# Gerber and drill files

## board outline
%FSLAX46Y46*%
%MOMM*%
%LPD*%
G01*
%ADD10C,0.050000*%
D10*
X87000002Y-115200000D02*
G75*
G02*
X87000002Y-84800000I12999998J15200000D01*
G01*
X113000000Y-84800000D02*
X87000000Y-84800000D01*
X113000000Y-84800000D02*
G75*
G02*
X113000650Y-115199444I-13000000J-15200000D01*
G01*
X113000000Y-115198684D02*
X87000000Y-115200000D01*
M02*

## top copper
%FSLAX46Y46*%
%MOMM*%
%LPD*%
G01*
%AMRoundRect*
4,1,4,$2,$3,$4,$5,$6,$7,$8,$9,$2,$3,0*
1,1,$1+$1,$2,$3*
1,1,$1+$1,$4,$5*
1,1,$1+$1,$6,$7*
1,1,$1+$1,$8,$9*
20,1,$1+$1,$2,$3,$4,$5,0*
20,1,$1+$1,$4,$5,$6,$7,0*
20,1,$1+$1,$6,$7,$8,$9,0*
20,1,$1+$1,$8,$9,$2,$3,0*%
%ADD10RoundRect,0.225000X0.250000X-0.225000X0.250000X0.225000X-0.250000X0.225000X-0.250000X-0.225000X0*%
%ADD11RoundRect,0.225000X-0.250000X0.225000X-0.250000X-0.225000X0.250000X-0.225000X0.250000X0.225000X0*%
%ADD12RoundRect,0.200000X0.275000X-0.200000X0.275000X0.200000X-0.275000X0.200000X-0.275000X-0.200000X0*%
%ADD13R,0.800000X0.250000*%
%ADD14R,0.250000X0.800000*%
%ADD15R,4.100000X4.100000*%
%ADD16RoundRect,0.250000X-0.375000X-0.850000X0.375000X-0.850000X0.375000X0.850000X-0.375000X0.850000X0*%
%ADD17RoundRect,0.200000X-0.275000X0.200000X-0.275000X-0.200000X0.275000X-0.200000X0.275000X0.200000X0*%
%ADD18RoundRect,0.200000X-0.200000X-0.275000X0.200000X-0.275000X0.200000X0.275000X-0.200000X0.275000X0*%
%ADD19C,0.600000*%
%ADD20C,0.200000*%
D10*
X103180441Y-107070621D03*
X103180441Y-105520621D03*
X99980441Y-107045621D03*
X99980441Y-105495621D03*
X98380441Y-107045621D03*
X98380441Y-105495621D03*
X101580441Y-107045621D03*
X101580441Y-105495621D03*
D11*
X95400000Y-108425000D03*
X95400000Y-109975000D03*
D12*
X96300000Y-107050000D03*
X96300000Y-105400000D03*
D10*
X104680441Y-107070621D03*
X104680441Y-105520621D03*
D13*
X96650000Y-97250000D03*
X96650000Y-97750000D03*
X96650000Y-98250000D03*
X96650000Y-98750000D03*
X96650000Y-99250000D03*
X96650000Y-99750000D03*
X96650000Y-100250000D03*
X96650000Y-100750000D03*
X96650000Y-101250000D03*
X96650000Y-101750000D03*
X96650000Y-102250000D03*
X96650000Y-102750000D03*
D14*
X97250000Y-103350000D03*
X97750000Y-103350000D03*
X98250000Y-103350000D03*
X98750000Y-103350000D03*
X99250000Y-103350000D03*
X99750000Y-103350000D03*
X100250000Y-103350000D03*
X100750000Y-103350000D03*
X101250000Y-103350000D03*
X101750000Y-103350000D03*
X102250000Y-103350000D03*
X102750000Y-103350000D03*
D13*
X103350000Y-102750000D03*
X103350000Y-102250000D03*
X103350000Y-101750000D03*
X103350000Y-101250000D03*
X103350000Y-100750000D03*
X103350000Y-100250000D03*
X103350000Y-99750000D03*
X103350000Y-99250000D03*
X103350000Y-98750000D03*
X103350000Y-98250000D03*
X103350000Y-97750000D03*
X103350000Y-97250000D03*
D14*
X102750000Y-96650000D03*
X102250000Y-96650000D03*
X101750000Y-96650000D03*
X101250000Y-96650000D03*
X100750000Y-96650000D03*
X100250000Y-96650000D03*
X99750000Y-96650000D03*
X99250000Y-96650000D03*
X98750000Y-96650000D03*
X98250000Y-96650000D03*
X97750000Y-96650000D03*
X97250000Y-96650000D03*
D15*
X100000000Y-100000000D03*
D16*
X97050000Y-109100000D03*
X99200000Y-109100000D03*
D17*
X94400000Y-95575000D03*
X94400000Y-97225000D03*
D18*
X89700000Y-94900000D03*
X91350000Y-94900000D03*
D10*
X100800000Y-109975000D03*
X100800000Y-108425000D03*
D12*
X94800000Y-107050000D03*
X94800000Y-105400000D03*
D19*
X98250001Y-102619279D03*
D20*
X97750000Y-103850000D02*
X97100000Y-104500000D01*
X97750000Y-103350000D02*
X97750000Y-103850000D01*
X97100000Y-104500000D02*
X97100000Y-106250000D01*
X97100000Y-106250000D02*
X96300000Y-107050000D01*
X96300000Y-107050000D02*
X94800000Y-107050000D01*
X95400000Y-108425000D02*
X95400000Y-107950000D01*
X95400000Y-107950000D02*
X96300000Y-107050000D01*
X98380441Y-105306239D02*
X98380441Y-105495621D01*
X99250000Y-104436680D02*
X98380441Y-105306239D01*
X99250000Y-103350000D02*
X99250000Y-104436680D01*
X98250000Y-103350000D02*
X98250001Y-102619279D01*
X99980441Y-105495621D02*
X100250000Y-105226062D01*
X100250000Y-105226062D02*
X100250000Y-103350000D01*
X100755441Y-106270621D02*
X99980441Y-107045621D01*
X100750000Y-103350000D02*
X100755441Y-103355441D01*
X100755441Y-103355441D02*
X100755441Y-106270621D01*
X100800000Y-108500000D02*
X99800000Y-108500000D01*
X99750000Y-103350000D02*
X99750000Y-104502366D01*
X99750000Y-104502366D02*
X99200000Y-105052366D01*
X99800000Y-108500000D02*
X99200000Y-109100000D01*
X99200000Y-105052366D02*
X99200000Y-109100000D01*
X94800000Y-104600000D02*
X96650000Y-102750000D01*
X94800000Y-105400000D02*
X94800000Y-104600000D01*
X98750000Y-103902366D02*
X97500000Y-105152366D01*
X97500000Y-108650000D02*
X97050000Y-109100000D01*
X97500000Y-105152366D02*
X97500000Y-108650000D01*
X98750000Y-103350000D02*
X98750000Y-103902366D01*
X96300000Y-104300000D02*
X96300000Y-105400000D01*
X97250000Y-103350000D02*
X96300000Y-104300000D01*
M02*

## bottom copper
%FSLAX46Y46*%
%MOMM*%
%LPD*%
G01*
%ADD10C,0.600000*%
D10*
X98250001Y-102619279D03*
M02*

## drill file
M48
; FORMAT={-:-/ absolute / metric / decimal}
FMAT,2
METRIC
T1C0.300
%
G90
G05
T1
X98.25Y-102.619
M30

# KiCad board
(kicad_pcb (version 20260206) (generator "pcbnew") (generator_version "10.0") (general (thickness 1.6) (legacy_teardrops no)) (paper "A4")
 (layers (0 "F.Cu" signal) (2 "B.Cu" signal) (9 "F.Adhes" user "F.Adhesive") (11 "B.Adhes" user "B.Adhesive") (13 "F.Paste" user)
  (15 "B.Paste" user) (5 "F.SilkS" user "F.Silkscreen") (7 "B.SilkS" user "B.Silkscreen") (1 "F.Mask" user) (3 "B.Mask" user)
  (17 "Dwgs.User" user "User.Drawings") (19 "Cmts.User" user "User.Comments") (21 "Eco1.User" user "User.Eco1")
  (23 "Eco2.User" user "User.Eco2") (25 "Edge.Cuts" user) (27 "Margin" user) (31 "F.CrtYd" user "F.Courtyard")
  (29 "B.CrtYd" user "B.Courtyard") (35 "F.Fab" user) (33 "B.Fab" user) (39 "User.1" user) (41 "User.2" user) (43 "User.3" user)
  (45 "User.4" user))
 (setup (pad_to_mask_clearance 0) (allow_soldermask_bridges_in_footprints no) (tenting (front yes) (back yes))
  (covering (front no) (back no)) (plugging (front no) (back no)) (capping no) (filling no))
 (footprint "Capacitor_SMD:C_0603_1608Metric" (layer "F.Cu") (at 103.180441 106.295621 90)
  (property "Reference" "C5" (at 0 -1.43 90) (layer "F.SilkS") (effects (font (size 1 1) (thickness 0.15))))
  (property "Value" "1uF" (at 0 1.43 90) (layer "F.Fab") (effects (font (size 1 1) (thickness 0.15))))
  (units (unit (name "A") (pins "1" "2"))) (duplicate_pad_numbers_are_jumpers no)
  (pad "1" smd roundrect (at -0.775 0 90) (size 0.9 0.95) (layers "F.Cu" "F.Mask" "F.Paste") (roundrect_rratio 0.25) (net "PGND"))
  (pad "2" smd roundrect (at 0.775 0 90) (size 0.9 0.95) (layers "F.Cu" "F.Mask" "F.Paste") (roundrect_rratio 0.25) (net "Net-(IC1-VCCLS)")))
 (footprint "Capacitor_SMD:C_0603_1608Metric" (layer "F.Cu") (at 99.980441 106.270621 90)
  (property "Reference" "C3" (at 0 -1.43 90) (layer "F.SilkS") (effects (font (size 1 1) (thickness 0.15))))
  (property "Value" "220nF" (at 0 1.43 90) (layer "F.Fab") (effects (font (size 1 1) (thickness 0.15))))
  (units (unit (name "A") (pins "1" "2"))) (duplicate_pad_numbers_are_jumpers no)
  (pad "1" smd roundrect (at -0.775 0 90) (size 0.9 0.95) (layers "F.Cu" "F.Mask" "F.Paste") (roundrect_rratio 0.25) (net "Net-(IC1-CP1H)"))
  (pad "2" smd roundrect (at 0.775 0 90) (size 0.9 0.95) (layers "F.Cu" "F.Mask" "F.Paste") (roundrect_rratio 0.25) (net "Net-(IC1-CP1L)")))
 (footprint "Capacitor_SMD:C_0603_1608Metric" (layer "F.Cu") (at 98.380441 106.270621 90)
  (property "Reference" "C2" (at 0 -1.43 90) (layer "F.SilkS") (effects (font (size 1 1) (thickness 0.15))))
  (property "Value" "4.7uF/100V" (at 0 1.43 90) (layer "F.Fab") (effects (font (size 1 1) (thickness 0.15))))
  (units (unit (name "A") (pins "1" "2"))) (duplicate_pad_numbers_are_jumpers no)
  (pad "1" smd roundrect (at -0.775 0 90) (size 0.9 0.95) (layers "F.Cu" "F.Mask" "F.Paste") (roundrect_rratio 0.25) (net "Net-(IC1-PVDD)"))
  (pad "2" smd roundrect (at 0.775 0 90) (size 0.9 0.95) (layers "F.Cu" "F.Mask" "F.Paste") (roundrect_rratio 0.25) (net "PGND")))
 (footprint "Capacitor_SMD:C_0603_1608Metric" (layer "F.Cu") (at 101.580441 106.270621 90)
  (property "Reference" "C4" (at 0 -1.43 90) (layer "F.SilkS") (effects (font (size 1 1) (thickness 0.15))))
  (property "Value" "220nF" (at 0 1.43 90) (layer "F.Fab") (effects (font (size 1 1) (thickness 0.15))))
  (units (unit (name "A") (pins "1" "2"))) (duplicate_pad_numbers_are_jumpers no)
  (pad "1" smd roundrect (at -0.775 0 90) (size 0.9 0.95) (layers "F.Cu" "F.Mask" "F.Paste") (roundrect_rratio 0.25) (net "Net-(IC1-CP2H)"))
  (pad "2" smd roundrect (at 0.775 0 90) (size 0.9 0.95) (layers "F.Cu" "F.Mask" "F.Paste") (roundrect_rratio 0.25) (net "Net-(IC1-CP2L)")))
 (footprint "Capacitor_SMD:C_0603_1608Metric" (layer "F.Cu") (at 95.4 109.2 -90)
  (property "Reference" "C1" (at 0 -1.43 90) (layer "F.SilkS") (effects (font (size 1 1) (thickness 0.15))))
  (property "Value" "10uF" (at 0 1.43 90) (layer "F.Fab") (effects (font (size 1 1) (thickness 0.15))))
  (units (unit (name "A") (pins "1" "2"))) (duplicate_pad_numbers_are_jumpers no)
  (pad "1" smd roundrect (at -0.775 0 270) (size 0.9 0.95) (layers "F.Cu" "F.Mask" "F.Paste") (roundrect_rratio 0.25) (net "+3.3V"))
  (pad "2" smd roundrect (at 0.775 0 270) (size 0.9 0.95) (layers "F.Cu" "F.Mask" "F.Paste") (roundrect_rratio 0.25) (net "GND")))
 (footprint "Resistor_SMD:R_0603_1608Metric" (layer "F.Cu") (at 96.3 106.225 90)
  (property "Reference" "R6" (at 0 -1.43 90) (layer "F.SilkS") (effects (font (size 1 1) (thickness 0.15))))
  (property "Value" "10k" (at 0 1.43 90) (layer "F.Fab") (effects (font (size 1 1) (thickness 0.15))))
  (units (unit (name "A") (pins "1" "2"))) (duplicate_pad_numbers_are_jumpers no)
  (pad "1" smd roundrect (at -0.825 0 90) (size 0.8 0.95) (layers "F.Cu" "F.Mask" "F.Paste") (roundrect_rratio 0.25) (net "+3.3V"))
  (pad "2" smd roundrect (at 0.825 0 90) (size 0.8 0.95) (layers "F.Cu" "F.Mask" "F.Paste") (roundrect_rratio 0.25) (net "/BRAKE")))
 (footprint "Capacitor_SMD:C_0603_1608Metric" (layer "F.Cu") (at 104.680441 106.295621 90)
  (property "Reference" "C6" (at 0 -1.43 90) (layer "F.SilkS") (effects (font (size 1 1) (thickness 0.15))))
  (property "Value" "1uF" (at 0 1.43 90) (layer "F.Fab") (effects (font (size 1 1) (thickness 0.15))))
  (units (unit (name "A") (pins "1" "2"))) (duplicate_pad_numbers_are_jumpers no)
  (pad "1" smd roundrect (at -0.775 0 90) (size 0.9 0.95) (layers "F.Cu" "F.Mask" "F.Paste") (roundrect_rratio 0.25) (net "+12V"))
  (pad "2" smd roundrect (at 0.775 0 90) (size 0.9 0.95) (layers "F.Cu" "F.Mask" "F.Paste") (roundrect_rratio 0.25) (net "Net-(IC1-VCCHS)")))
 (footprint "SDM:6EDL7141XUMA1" (layer "F.Cu") (at 100 100)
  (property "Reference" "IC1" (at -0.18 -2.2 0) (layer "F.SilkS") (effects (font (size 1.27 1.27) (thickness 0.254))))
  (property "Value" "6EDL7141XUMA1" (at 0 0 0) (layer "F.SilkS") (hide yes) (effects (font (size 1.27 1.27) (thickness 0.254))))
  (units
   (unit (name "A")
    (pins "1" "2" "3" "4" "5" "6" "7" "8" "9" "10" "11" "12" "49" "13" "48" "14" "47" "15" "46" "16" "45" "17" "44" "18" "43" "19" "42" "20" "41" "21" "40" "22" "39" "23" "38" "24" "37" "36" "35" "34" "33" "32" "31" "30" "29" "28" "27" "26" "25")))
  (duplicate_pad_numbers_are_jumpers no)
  (pad "1" smd rect (at -3.35 -2.75 90) (size 0.25 0.8) (layers "F.Cu" "F.Mask" "F.Paste") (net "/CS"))
  (pad "2" smd rect (at -3.35 -2.25 90) (size 0.25 0.8) (layers "F.Cu" "F.Mask" "F.Paste") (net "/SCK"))
  (pad "3" smd rect (at -3.35 -1.75 90) (size 0.25 0.8) (layers "F.Cu" "F.Mask" "F.Paste") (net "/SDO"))
  (pad "4" smd rect (at -3.35 -1.25 90) (size 0.25 0.8) (layers "F.Cu" "F.Mask" "F.Paste") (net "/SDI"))
  (pad "5" smd rect (at -3.35 -0.75 90) (size 0.25 0.8) (layers "F.Cu" "F.Mask" "F.Paste") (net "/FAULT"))
  (pad "6" smd rect (at -3.35 -0.25 90) (size 0.25 0.8) (layers "F.Cu" "F.Mask" "F.Paste") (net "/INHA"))
  (pad "7" smd rect (at -3.35 0.25 90) (size 0.25 0.8) (layers "F.Cu" "F.Mask" "F.Paste") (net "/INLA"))
  (pad "8" smd rect (at -3.35 0.75 90) (size 0.25 0.8) (layers "F.Cu" "F.Mask" "F.Paste") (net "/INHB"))
  (pad "9" smd rect (at -3.35 1.25 90) (size 0.25 0.8) (layers "F.Cu" "F.Mask" "F.Paste") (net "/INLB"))
  (pad "10" smd rect (at -3.35 1.75 90) (size 0.25 0.8) (layers "F.Cu" "F.Mask" "F.Paste") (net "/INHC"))
  (pad "11" smd rect (at -3.35 2.25 90) (size 0.25 0.8) (layers "F.Cu" "F.Mask" "F.Paste") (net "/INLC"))
  (pad "12" smd rect (at -3.35 2.75 90) (size 0.25 0.8) (layers "F.Cu" "F.Mask" "F.Paste") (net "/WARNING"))
  (pad "13" smd rect (at -2.75 3.35) (size 0.25 0.8) (layers "F.Cu" "F.Mask" "F.Paste") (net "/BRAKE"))
  (pad "14" smd rect (at -2.25 3.35) (size 0.25 0.8) (layers "F.Cu" "F.Mask" "F.Paste") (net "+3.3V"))
  (pad "15" smd rect (at -1.75 3.35) (size 0.25 0.8) (layers "F.Cu" "F.Mask" "F.Paste") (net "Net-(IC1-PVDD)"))
  (pad "16" smd rect (at -1.25 3.35) (size 0.25 0.8) (layers "F.Cu" "F.Mask" "F.Paste") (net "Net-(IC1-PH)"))
  (pad "17" smd rect (at -0.75 3.35) (size 0.25 0.8) (layers "F.Cu" "F.Mask" "F.Paste") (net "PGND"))
  (pad "18" smd rect (at -0.25 3.35) (size 0.25 0.8) (layers "F.Cu" "F.Mask" "F.Paste") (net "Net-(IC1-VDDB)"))
  (pad "19" smd rect (at 0.25 3.35) (size 0.25 0.8) (layers "F.Cu" "F.Mask" "F.Paste") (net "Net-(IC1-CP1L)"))
  (pad "20" smd rect (at 0.75 3.35) (size 0.25 0.8) (layers "F.Cu" "F.Mask" "F.Paste") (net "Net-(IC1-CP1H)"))
  (pad "21" smd rect (at 1.25 3.35) (size 0.25 0.8) (layers "F.Cu" "F.Mask" "F.Paste") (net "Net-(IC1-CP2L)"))
  (pad "22" smd rect (at 1.75 3.35) (size 0.25 0.8) (layers "F.Cu" "F.Mask" "F.Paste") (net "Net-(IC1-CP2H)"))
  (pad "23" smd rect (at 2.25 3.35) (size 0.25 0.8) (layers "F.Cu" "F.Mask" "F.Paste") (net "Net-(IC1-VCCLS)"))
  (pad "24" smd rect (at 2.75 3.35) (size 0.25 0.8) (layers "F.Cu" "F.Mask" "F.Paste") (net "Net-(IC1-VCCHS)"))
  (pad "25" smd rect (at 3.35 2.75 90) (size 0.25 0.8) (layers "F.Cu" "F.Mask" "F.Paste") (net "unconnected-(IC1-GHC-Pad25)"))
  (pad "26" smd rect (at 3.35 2.25 90) (size 0.25 0.8) (layers "F.Cu" "F.Mask" "F.Paste") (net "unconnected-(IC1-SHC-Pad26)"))
  (pad "27" smd rect (at 3.35 1.75 90) (size 0.25 0.8) (layers "F.Cu" "F.Mask" "F.Paste") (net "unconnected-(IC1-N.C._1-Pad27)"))
  (pad "28" smd rect (at 3.35 1.25 90) (size 0.25 0.8) (layers "F.Cu" "F.Mask" "F.Paste") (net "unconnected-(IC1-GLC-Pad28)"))
  (pad "29" smd rect (at 3.35 0.75 90) (size 0.25 0.8) (layers "F.Cu" "F.Mask" "F.Paste") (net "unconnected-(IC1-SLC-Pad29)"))
  (pad "30" smd rect (at 3.35 0.25 90) (size 0.25 0.8) (layers "F.Cu" "F.Mask" "F.Paste") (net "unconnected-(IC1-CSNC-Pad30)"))
  (pad "31" smd rect (at 3.35 -0.25 90) (size 0.25 0.8) (layers "F.Cu" "F.Mask" "F.Paste") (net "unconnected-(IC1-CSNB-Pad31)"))
  (pad "32" smd rect (at 3.35 -0.75 90) (size 0.25 0.8) (layers "F.Cu" "F.Mask" "F.Paste") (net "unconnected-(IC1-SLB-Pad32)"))
  (pad "33" smd rect (at 3.35 -1.25 90) (size 0.25 0.8) (layers "F.Cu" "F.Mask" "F.Paste") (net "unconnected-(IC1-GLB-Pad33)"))
  (pad "34" smd rect (at 3.35 -1.75 90) (size 0.25 0.8) (layers "F.Cu" "F.Mask" "F.Paste") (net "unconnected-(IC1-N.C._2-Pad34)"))
  (pad "35" smd rect (at 3.35 -2.25 90) (size 0.25 0.8) (layers "F.Cu" "F.Mask" "F.Paste") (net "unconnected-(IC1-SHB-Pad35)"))
  (pad "36" smd rect (at 3.35 -2.75 90) (size 0.25 0.8) (layers "F.Cu" "F.Mask" "F.Paste") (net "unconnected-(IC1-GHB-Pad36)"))
  (pad "37" smd rect (at 2.75 -3.35) (size 0.25 0.8) (layers "F.Cu" "F.Mask" "F.Paste") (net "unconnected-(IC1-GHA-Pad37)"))
  (pad "38" smd rect (at 2.25 -3.35) (size 0.25 0.8) (layers "F.Cu" "F.Mask" "F.Paste") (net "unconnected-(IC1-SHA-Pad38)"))
  (pad "39" smd rect (at 1.75 -3.35) (size 0.25 0.8) (layers "F.Cu" "F.Mask" "F.Paste") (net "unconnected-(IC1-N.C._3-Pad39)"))
  (pad "40" smd rect (at 1.25 -3.35) (size 0.25 0.8) (layers "F.Cu" "F.Mask" "F.Paste") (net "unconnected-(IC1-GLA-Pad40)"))
  (pad "41" smd rect (at 0.75 -3.35) (size 0.25 0.8) (layers "F.Cu" "F.Mask" "F.Paste") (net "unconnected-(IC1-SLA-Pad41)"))
  (pad "42" smd rect (at 0.25 -3.35) (size 0.25 0.8) (layers "F.Cu" "F.Mask" "F.Paste") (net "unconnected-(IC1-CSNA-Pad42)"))
  (pad "43" smd rect (at -0.25 -3.35) (size 0.25 0.8) (layers "F.Cu" "F.Mask" "F.Paste") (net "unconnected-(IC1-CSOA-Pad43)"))
  (pad "44" smd rect (at -0.75 -3.35) (size 0.25 0.8) (layers "F.Cu" "F.Mask" "F.Paste") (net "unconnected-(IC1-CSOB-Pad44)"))
  (pad "45" smd rect (at -1.25 -3.35) (size 0.25 0.8) (layers "F.Cu" "F.Mask" "F.Paste") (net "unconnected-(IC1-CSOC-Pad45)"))
  (pad "46" smd rect (at -1.75 -3.35) (size 0.25 0.8) (layers "F.Cu" "F.Mask" "F.Paste") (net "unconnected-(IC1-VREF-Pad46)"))
  (pad "47" smd rect (at -2.25 -3.35) (size 0.25 0.8) (layers "F.Cu" "F.Mask" "F.Paste") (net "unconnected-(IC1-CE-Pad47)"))
  (pad "48" smd rect (at -2.75 -3.35) (size 0.25 0.8) (layers "F.Cu" "F.Mask" "F.Paste") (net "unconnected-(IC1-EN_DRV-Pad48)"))
  (pad "49" smd rect (at 0 0 90) (size 4.1 4.1) (layers "F.Cu" "F.Mask" "F.Paste") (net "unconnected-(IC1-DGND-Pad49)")))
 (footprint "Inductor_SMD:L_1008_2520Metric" (layer "F.Cu") (at 98.125 109.1)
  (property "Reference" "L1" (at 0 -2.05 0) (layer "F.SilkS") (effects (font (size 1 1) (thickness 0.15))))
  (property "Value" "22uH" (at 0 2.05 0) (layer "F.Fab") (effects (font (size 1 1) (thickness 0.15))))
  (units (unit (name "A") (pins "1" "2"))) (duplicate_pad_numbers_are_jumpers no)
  (pad "1" smd roundrect (at -1.075 0) (size 1.25 2.2) (layers "F.Cu" "F.Mask" "F.Paste") (roundrect_rratio 0.2) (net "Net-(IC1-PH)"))
  (pad "2" smd roundrect (at 1.075 0) (size 1.25 2.2) (layers "F.Cu" "F.Mask" "F.Paste") (roundrect_rratio 0.2) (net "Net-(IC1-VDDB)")))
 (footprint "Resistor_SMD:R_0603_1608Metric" (layer "F.Cu") (at 94.4 96.4 -90)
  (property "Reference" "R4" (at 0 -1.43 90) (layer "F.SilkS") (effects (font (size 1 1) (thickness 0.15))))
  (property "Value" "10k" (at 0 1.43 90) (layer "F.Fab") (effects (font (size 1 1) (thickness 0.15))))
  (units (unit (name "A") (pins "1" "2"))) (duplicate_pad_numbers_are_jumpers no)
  (pad "1" smd roundrect (at -0.825 0 270) (size 0.8 0.95) (layers "F.Cu" "F.Mask" "F.Paste") (roundrect_rratio 0.25) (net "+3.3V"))
  (pad "2" smd roundrect (at 0.825 0 270) (size 0.8 0.95) (layers "F.Cu" "F.Mask" "F.Paste") (roundrect_rratio 0.25) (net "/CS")))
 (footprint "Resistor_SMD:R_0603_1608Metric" (layer "F.Cu") (at 90.525 94.9)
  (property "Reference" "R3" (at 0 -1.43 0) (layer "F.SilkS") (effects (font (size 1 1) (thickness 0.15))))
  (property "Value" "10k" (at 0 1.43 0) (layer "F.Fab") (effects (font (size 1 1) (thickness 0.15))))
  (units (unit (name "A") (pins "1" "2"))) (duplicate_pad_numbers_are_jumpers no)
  (pad "1" smd roundrect (at -0.825 0) (size 0.8 0.95) (layers "F.Cu" "F.Mask" "F.Paste") (roundrect_rratio 0.25) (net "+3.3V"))
  (pad "2" smd roundrect (at 0.825 0) (size 0.8 0.95) (layers "F.Cu" "F.Mask" "F.Paste") (roundrect_rratio 0.25) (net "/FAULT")))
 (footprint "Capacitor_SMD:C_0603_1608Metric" (layer "F.Cu") (at 100.8 109.2 90)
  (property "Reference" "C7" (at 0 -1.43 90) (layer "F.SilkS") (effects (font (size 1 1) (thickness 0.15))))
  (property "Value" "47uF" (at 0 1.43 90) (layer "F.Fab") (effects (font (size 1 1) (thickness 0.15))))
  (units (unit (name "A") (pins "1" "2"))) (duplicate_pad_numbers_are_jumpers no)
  (pad "1" smd roundrect (at -0.775 0 90) (size 0.9 0.95) (layers "F.Cu" "F.Mask" "F.Paste") (roundrect_rratio 0.25) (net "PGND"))
  (pad "2" smd roundrect (at 0.775 0 90) (size 0.9 0.95) (layers "F.Cu" "F.Mask" "F.Paste") (roundrect_rratio 0.25) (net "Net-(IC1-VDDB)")))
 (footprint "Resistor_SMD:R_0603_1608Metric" (layer "F.Cu") (at 94.8 106.225 90)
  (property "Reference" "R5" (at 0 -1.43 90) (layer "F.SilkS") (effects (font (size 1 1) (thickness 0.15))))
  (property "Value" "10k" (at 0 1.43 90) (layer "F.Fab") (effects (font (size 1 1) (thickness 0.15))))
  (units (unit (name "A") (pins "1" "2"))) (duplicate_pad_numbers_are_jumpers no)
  (pad "1" smd roundrect (at -0.825 0 90) (size 0.8 0.95) (layers "F.Cu" "F.Mask" "F.Paste") (roundrect_rratio 0.25) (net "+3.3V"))
  (pad "2" smd roundrect (at 0.825 0 90) (size 0.8 0.95) (layers "F.Cu" "F.Mask" "F.Paste") (roundrect_rratio 0.25) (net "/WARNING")))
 (gr_arc (start 87.000002 115.2) (mid 79.999001 100) (end 87.000002 84.8) (stroke (width 0.05) (type default)) (layer "Edge.Cuts"))
 (gr_line (start 113 84.8) (end 87 84.8) (stroke (width 0.05) (type default)) (layer "Edge.Cuts"))
 (gr_arc (start 113 84.8) (mid 120.001 99.999572) (end 113.00065 115.199444) (stroke (width 0.05) (type default)) (layer "Edge.Cuts"))
 (gr_line (start 113 115.198684) (end 87 115.2) (stroke (width 0.05) (type default)) (layer "Edge.Cuts"))
 (segment (start 97.75 103.85) (end 97.1 104.5) (width 0.2) (layer "F.Cu") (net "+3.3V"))
 (segment (start 97.75 103.35) (end 97.75 103.85) (width 0.2) (layer "F.Cu") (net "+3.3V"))
 (segment (start 97.1 104.5) (end 97.1 106.25) (width 0.2) (layer "F.Cu") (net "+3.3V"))
 (segment (start 97.1 106.25) (end 96.3 107.05) (width 0.2) (layer "F.Cu") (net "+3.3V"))
 (segment (start 96.3 107.05) (end 94.8 107.05) (width 0.2) (layer "F.Cu") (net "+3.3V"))
 (segment (start 95.4 108.425) (end 95.4 107.95) (width 0.2) (layer "F.Cu") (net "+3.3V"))
 (segment (start 95.4 107.95) (end 96.3 107.05) (width 0.2) (layer "F.Cu") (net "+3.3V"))
 (segment (start 98.380441 105.306239) (end 98.380441 105.495621) (width 0.2) (layer "F.Cu") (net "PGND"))
 (segment (start 99.25 104.43668) (end 98.380441 105.306239) (width 0.2) (layer "F.Cu") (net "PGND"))
 (segment (start 99.25 103.35) (end 99.25 104.43668) (width 0.2) (layer "F.Cu") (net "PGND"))
 (segment (start 98.25 103.35) (end 98.250001 102.619279) (width 0.2) (layer "F.Cu") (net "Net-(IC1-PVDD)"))
 (via (at 98.250001 102.619279) (size 0.6) (drill 0.3) (layers "F.Cu" "B.Cu") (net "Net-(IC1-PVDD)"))
 (segment (start 99.980441 105.495621) (end 100.25 105.226062) (width 0.2) (layer "F.Cu") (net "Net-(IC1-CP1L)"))
 (segment (start 100.25 105.226062) (end 100.25 103.35) (width 0.2) (layer "F.Cu") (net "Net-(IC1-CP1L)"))
 (segment (start 100.755441 106.270621) (end 99.980441 107.045621) (width 0.2) (layer "F.Cu") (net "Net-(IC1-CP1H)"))
 (segment (start 100.75 103.35) (end 100.755441 103.355441) (width 0.2) (layer "F.Cu") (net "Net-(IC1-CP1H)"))
 (segment (start 100.755441 103.355441) (end 100.755441 106.270621) (width 0.2) (layer "F.Cu") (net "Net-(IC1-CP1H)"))
 (segment (start 100.8 108.5) (end 99.8 108.5) (width 0.2) (layer "F.Cu") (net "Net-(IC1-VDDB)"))
 (segment (start 99.75 103.35) (end 99.75 104.502366) (width 0.2) (layer "F.Cu") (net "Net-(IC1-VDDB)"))
 (segment (start 99.75 104.502366) (end 99.2 105.052366) (width 0.2) (layer "F.Cu") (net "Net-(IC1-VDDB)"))
 (segment (start 99.8 108.5) (end 99.2 109.1) (width 0.2) (layer "F.Cu") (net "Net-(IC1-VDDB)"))
 (segment (start 99.2 105.052366) (end 99.2 109.1) (width 0.2) (layer "F.Cu") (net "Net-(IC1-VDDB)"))
 (segment (start 94.8 104.6) (end 96.65 102.75) (width 0.2) (layer "F.Cu") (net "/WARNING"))
 (segment (start 94.8 105.4) (end 94.8 104.6) (width 0.2) (layer "F.Cu") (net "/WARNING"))
 (segment (start 98.75 103.902366) (end 97.5 105.152366) (width 0.2) (layer "F.Cu") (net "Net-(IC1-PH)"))
 (segment (start 97.5 108.65) (end 97.05 109.1) (width 0.2) (layer "F.Cu") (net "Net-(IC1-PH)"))
 (segment (start 97.5 105.152366) (end 97.5 108.65) (width 0.2) (layer "F.Cu") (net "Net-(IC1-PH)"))
 (segment (start 98.75 103.35) (end 98.75 103.902366) (width 0.2) (layer "F.Cu") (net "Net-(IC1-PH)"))
 (segment (start 96.3 104.3) (end 96.3 105.4) (width 0.2) (layer "F.Cu") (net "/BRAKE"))
 (segment (start 97.25 103.35) (end 96.3 104.3) (width 0.2) (layer "F.Cu") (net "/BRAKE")))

